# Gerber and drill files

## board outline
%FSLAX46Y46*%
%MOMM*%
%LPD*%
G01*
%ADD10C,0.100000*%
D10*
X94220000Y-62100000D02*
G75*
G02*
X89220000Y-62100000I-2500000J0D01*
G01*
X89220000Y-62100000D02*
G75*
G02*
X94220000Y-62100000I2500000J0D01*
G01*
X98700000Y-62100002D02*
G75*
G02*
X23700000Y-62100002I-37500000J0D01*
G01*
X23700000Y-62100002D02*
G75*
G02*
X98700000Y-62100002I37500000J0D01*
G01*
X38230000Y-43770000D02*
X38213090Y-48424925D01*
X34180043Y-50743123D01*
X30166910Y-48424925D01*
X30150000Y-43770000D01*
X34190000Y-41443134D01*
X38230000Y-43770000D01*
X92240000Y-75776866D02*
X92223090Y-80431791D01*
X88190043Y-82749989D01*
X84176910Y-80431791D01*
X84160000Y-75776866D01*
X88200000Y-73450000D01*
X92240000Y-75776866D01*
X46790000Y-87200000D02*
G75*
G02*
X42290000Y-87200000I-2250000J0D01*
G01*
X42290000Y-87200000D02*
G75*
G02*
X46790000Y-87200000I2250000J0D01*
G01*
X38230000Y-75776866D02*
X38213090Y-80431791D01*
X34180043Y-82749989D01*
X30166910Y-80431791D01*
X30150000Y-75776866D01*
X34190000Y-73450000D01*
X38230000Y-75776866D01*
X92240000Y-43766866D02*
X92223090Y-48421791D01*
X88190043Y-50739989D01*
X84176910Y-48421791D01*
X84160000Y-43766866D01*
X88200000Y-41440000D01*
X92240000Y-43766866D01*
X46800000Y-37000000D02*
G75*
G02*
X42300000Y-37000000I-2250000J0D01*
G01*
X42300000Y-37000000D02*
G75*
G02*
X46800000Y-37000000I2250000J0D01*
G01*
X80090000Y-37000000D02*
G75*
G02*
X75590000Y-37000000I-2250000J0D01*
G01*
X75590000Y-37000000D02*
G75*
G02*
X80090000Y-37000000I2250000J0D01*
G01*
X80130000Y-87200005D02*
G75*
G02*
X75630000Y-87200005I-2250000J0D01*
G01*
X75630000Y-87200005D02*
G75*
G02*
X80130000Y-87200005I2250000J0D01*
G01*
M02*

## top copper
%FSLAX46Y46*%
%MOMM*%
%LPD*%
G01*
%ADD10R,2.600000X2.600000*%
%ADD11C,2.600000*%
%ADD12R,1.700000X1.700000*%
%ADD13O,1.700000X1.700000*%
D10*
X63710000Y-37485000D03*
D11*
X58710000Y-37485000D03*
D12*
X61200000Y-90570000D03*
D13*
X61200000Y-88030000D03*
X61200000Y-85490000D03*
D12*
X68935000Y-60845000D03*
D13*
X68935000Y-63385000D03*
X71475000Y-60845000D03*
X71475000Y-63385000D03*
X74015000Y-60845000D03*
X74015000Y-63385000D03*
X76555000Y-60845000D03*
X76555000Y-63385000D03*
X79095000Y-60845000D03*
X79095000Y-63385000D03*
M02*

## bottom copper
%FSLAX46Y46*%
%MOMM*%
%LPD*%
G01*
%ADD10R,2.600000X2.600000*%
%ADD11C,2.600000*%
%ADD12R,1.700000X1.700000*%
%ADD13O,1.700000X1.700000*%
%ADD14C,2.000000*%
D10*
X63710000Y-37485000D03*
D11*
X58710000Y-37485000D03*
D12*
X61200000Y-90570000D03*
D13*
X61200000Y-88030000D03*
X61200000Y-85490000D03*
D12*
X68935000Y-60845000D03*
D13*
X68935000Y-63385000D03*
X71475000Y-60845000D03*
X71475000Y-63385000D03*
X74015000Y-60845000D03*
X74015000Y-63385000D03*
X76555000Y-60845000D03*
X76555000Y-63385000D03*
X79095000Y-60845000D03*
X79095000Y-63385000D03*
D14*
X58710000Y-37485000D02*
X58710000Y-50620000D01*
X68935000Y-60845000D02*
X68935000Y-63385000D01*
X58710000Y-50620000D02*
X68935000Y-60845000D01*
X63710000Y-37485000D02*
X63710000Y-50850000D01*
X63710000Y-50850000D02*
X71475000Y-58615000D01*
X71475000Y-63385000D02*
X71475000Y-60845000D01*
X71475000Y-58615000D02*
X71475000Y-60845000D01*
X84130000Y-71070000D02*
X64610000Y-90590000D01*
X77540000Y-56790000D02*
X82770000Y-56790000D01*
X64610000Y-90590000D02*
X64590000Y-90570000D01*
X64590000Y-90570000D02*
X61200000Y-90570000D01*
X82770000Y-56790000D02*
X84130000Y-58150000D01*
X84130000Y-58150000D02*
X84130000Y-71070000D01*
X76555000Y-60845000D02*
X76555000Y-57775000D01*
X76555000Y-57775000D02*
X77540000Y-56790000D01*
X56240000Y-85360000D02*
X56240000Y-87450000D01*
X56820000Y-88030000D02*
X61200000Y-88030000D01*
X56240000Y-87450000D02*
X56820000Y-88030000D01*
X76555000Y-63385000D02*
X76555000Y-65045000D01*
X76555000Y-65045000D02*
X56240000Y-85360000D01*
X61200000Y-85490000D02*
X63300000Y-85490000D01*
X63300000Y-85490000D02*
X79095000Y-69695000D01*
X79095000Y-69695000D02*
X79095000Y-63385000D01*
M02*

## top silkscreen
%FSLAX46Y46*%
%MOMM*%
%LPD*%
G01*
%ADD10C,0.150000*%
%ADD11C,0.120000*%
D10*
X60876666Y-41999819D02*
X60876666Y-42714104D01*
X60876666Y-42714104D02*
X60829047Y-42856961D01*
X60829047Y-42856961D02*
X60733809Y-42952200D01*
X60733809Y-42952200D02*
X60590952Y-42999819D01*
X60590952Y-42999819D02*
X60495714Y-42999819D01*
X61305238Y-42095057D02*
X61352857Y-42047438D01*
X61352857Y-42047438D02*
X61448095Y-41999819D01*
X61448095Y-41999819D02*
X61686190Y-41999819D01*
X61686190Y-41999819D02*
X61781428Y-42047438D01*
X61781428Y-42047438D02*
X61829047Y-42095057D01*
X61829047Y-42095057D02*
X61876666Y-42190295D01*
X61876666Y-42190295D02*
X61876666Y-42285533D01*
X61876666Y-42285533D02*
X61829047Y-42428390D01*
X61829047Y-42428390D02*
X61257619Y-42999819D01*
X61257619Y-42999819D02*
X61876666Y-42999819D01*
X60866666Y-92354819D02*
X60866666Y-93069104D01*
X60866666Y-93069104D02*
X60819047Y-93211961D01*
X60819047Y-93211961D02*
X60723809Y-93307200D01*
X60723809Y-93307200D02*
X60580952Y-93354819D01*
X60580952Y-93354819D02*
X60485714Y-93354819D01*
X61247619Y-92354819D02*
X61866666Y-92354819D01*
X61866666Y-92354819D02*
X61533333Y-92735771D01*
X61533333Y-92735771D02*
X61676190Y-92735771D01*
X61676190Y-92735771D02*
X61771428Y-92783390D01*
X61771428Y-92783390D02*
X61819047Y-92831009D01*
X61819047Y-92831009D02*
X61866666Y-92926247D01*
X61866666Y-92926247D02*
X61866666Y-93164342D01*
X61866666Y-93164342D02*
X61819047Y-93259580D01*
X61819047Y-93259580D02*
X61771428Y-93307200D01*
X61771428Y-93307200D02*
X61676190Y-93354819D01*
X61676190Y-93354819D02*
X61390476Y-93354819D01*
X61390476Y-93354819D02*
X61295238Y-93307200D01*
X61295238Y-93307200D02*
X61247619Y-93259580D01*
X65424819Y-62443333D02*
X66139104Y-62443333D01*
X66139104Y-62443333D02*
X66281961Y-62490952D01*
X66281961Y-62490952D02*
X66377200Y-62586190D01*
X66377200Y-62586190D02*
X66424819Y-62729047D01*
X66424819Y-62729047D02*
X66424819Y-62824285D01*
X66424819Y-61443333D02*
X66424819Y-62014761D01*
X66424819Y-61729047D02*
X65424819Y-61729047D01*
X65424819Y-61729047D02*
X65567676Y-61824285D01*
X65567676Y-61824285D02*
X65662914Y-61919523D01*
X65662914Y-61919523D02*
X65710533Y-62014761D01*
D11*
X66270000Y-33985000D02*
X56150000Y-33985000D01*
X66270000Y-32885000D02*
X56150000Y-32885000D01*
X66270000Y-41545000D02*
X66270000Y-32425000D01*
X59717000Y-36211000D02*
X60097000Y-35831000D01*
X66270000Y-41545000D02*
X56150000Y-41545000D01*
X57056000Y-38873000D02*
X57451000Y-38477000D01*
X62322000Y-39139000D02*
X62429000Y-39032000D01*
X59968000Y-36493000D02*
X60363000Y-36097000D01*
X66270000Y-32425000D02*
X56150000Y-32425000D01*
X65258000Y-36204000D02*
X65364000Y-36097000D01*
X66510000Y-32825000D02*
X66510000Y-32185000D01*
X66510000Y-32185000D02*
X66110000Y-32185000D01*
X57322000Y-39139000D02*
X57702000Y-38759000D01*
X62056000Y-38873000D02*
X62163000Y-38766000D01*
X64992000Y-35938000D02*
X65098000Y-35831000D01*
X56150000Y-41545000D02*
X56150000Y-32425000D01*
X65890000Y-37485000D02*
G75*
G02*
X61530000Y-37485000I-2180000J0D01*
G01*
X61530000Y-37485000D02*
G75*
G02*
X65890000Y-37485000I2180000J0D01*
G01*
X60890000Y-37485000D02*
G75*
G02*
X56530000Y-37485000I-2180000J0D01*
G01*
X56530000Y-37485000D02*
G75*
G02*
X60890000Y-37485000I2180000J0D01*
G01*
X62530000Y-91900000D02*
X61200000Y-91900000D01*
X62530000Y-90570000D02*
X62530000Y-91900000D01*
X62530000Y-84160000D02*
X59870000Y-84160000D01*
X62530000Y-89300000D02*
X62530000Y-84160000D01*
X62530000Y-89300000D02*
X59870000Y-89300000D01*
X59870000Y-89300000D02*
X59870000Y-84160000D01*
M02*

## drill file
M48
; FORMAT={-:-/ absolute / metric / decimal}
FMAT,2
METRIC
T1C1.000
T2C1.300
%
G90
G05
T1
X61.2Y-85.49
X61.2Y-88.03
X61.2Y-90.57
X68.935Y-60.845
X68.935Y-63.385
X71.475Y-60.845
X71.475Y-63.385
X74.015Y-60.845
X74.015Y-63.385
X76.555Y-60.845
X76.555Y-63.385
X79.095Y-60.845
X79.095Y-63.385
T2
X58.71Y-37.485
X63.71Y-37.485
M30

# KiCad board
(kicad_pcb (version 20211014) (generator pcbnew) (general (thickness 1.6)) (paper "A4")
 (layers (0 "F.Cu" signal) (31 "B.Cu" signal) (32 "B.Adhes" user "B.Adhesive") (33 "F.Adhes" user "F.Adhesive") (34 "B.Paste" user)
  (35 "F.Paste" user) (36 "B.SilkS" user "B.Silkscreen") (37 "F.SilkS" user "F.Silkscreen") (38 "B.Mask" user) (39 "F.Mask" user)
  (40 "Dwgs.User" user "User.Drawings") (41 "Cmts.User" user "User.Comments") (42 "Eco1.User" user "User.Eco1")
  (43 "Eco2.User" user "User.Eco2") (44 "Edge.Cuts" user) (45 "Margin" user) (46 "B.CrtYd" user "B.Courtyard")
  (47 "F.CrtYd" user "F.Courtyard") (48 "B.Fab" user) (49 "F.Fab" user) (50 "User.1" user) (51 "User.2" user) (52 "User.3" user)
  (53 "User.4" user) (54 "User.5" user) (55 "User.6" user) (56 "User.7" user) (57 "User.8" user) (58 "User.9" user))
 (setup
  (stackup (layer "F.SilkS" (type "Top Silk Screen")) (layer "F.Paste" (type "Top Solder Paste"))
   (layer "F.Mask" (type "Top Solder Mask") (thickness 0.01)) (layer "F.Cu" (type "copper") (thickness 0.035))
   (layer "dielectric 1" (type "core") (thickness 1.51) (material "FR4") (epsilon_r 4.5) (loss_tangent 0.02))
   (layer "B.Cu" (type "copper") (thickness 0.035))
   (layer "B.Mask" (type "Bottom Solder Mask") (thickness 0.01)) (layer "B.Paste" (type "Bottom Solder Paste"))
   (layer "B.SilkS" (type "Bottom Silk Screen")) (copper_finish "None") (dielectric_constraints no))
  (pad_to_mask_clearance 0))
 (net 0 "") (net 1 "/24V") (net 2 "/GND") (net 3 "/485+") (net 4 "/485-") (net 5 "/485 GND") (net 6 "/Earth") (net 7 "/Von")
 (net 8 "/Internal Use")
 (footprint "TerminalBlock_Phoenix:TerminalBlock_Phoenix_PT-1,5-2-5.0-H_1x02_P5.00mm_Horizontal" (layer "F.Cu") (at 63.71 37.485 180)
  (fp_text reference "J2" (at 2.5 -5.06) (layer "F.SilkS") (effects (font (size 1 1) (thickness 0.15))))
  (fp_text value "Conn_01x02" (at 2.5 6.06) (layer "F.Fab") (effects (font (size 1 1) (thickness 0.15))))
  (fp_line (start -2.56 3.5) (end 7.56 3.5) (layer "F.SilkS") (width 0.12))
  (fp_line (start -2.56 4.6) (end 7.56 4.6) (layer "F.SilkS") (width 0.12))
  (fp_line (start -2.56 -4.06) (end -2.56 5.06) (layer "F.SilkS") (width 0.12))
  (fp_line (start 3.993 1.274) (end 3.613 1.654) (layer "F.SilkS") (width 0.12))
  (fp_line (start -2.56 -4.06) (end 7.56 -4.06) (layer "F.SilkS") (width 0.12))
  (fp_line (start 6.654 -1.388) (end 6.259 -0.992) (layer "F.SilkS") (width 0.12))
  (fp_line (start 1.388 -1.654) (end 1.281 -1.547) (layer "F.SilkS") (width 0.12))
  (fp_line (start 3.742 0.992) (end 3.347 1.388) (layer "F.SilkS") (width 0.12))
  (fp_line (start -2.56 5.06) (end 7.56 5.06) (layer "F.SilkS") (width 0.12))
  (fp_line (start -1.548 1.281) (end -1.654 1.388) (layer "F.SilkS") (width 0.12))
  (fp_line (start -2.8 4.66) (end -2.8 5.3) (layer "F.SilkS") (width 0.12))
  (fp_line (start -2.8 5.3) (end -2.4 5.3) (layer "F.SilkS") (width 0.12))
  (fp_line (start 6.388 -1.654) (end 6.008 -1.274) (layer "F.SilkS") (width 0.12))
  (fp_line (start 1.654 -1.388) (end 1.547 -1.281) (layer "F.SilkS") (width 0.12))
  (fp_line (start -1.282 1.547) (end -1.388 1.654) (layer "F.SilkS") (width 0.12))
  (fp_line (start 7.56 -4.06) (end 7.56 5.06) (layer "F.SilkS") (width 0.12))
  (fp_circle (center 0 0) (end 2.18 0) (layer "F.SilkS") (width 0.12) (fill none))
  (fp_circle (center 5 0) (end 7.18 0) (layer "F.SilkS") (width 0.12) (fill none))
  (pad "1" thru_hole rect (at 0 0 180) (size 2.6 2.6) (drill 1.3) (layers *.Cu *.Mask) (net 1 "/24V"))
  (pad "2" thru_hole circle (at 5 0 180) (size 2.6 2.6) (drill 1.3) (layers *.Cu *.Mask) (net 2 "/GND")))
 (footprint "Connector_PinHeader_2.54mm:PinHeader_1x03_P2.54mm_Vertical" (layer "F.Cu") (at 61.2 90.57 180)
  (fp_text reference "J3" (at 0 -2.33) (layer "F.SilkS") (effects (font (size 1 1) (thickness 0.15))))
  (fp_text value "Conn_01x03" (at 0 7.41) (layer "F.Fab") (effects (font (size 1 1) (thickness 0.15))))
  (fp_line (start -1.33 -1.33) (end 0 -1.33) (layer "F.SilkS") (width 0.12))
  (fp_line (start -1.33 0) (end -1.33 -1.33) (layer "F.SilkS") (width 0.12))
  (fp_line (start -1.33 6.41) (end 1.33 6.41) (layer "F.SilkS") (width 0.12))
  (fp_line (start -1.33 1.27) (end -1.33 6.41) (layer "F.SilkS") (width 0.12))
  (fp_line (start -1.33 1.27) (end 1.33 1.27) (layer "F.SilkS") (width 0.12))
  (fp_line (start 1.33 1.27) (end 1.33 6.41) (layer "F.SilkS") (width 0.12))
  (pad "1" thru_hole rect (at 0 0 180) (size 1.7 1.7) (drill 1) (layers *.Cu *.Mask) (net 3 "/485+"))
  (pad "2" thru_hole oval (at 0 2.54 180) (size 1.7 1.7) (drill 1) (layers *.Cu *.Mask) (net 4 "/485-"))
  (pad "3" thru_hole oval (at 0 5.08 180) (size 1.7 1.7) (drill 1) (layers *.Cu *.Mask) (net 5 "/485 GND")))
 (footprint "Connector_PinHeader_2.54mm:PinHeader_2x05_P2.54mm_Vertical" (layer "B.Cu") (at 68.935 60.845 -90)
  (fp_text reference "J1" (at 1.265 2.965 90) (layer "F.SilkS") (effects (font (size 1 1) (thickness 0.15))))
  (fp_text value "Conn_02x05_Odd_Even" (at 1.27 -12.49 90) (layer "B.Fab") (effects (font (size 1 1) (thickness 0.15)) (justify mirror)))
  (pad "1" thru_hole rect (at 0 0 270) (size 1.7 1.7) (drill 1) (layers *.Cu *.Mask) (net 2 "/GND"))
  (pad "2" thru_hole oval (at 2.54 0 270) (size 1.7 1.7) (drill 1) (layers *.Cu *.Mask) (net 2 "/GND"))
  (pad "3" thru_hole oval (at 0 -2.54 270) (size 1.7 1.7) (drill 1) (layers *.Cu *.Mask) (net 1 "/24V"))
  (pad "4" thru_hole oval (at 2.54 -2.54 270) (size 1.7 1.7) (drill 1) (layers *.Cu *.Mask) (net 1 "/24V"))
  (pad "5" thru_hole oval (at 0 -5.08 270) (size 1.7 1.7) (drill 1) (layers *.Cu *.Mask) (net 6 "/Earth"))
  (pad "6" thru_hole oval (at 2.54 -5.08 270) (size 1.7 1.7) (drill 1) (layers *.Cu *.Mask) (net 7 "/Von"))
  (pad "7" thru_hole oval (at 0 -7.62 270) (size 1.7 1.7) (drill 1) (layers *.Cu *.Mask) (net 3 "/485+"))
  (pad "8" thru_hole oval (at 2.54 -7.62 270) (size 1.7 1.7) (drill 1) (layers *.Cu *.Mask) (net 4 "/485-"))
  (pad "9" thru_hole oval (at 0 -10.16 270) (size 1.7 1.7) (drill 1) (layers *.Cu *.Mask) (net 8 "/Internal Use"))
  (pad "10" thru_hole oval (at 2.54 -10.16 270) (size 1.7 1.7) (drill 1) (layers *.Cu *.Mask) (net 5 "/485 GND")))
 (gr_circle (center 91.72 62.1) (end 94.22 62.1) (layer "Edge.Cuts") (width 0.1) (fill none))
 (gr_circle (center 61.2 62.100002) (end 98.7 62.100002) (layer "Edge.Cuts") (width 0.1) (fill none))
 (gr_poly
  (pts (xy 38.23 43.77) (xy 38.21309 48.424925) (xy 34.180043 50.743123) (xy 30.16691 48.424925) (xy 30.15 43.77) (xy 34.19 41.443134))
  (layer "Edge.Cuts") (width 0.1) (fill none))
 (gr_poly
  (pts (xy 92.24 75.776866) (xy 92.22309 80.431791) (xy 88.190043 82.749989) (xy 84.17691 80.431791) (xy 84.16 75.776866) (xy 88.2 73.45))
  (layer "Edge.Cuts") (width 0.1) (fill none))
 (gr_circle (center 44.54 87.2) (end 46.79 87.2) (layer "Edge.Cuts") (width 0.1) (fill none))
 (gr_poly
  (pts (xy 38.23 75.776866) (xy 38.21309 80.431791) (xy 34.180043 82.749989) (xy 30.16691 80.431791) (xy 30.15 75.776866) (xy 34.19 73.45))
  (layer "Edge.Cuts") (width 0.1) (fill none))
 (gr_poly
  (pts (xy 92.24 43.766866) (xy 92.22309 48.421791) (xy 88.190043 50.739989) (xy 84.17691 48.421791) (xy 84.16 43.766866) (xy 88.2 41.44))
  (layer "Edge.Cuts") (width 0.1) (fill none))
 (gr_circle (center 44.55 37) (end 46.8 37) (layer "Edge.Cuts") (width 0.1) (fill none))
 (gr_circle (center 77.84 37) (end 80.09 37) (layer "Edge.Cuts") (width 0.1) (fill none))
 (gr_circle (center 77.88 87.200005) (end 80.13 87.200005) (layer "Edge.Cuts") (width 0.1) (fill none))
 (segment (start 58.71 37.485) (end 58.71 50.62) (width 2) (layer "B.Cu") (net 2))
 (segment (start 68.935 60.845) (end 68.935 63.385) (width 2) (layer "B.Cu") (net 2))
 (segment (start 58.71 50.62) (end 68.935 60.845) (width 2) (layer "B.Cu") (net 2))
 (segment (start 63.71 37.485) (end 63.71 50.85) (width 2) (layer "B.Cu") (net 1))
 (segment (start 63.71 50.85) (end 71.475 58.615) (width 2) (layer "B.Cu") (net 1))
 (segment (start 71.475 63.385) (end 71.475 60.845) (width 2) (layer "B.Cu") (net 1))
 (segment (start 71.475 58.615) (end 71.475 60.845) (width 2) (layer "B.Cu") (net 1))
 (segment (start 84.13 71.07) (end 64.61 90.59) (width 2) (layer "B.Cu") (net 3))
 (segment (start 77.54 56.79) (end 82.77 56.79) (width 2) (layer "B.Cu") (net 3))
 (segment (start 64.61 90.59) (end 64.59 90.57) (width 2) (layer "B.Cu") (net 3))
 (segment (start 64.59 90.57) (end 61.2 90.57) (width 2) (layer "B.Cu") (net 3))
 (segment (start 82.77 56.79) (end 84.13 58.15) (width 2) (layer "B.Cu") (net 3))
 (segment (start 84.13 58.15) (end 84.13 71.07) (width 2) (layer "B.Cu") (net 3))
 (segment (start 76.555 60.845) (end 76.555 57.775) (width 2) (layer "B.Cu") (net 3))
 (segment (start 76.555 57.775) (end 77.54 56.79) (width 2) (layer "B.Cu") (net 3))
 (segment (start 56.24 85.36) (end 56.24 87.45) (width 2) (layer "B.Cu") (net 4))
 (segment (start 56.82 88.03) (end 61.2 88.03) (width 2) (layer "B.Cu") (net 4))
 (segment (start 56.24 87.45) (end 56.82 88.03) (width 2) (layer "B.Cu") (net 4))
 (segment (start 76.555 63.385) (end 76.555 65.045) (width 2) (layer "B.Cu") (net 4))
 (segment (start 76.555 65.045) (end 56.24 85.36) (width 2) (layer "B.Cu") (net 4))
 (segment (start 61.2 85.49) (end 63.3 85.49) (width 2) (layer "B.Cu") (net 5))
 (segment (start 63.3 85.49) (end 79.095 69.695) (width 2) (layer "B.Cu") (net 5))
 (segment (start 79.095 69.695) (end 79.095 63.385) (width 2) (layer "B.Cu") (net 5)))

